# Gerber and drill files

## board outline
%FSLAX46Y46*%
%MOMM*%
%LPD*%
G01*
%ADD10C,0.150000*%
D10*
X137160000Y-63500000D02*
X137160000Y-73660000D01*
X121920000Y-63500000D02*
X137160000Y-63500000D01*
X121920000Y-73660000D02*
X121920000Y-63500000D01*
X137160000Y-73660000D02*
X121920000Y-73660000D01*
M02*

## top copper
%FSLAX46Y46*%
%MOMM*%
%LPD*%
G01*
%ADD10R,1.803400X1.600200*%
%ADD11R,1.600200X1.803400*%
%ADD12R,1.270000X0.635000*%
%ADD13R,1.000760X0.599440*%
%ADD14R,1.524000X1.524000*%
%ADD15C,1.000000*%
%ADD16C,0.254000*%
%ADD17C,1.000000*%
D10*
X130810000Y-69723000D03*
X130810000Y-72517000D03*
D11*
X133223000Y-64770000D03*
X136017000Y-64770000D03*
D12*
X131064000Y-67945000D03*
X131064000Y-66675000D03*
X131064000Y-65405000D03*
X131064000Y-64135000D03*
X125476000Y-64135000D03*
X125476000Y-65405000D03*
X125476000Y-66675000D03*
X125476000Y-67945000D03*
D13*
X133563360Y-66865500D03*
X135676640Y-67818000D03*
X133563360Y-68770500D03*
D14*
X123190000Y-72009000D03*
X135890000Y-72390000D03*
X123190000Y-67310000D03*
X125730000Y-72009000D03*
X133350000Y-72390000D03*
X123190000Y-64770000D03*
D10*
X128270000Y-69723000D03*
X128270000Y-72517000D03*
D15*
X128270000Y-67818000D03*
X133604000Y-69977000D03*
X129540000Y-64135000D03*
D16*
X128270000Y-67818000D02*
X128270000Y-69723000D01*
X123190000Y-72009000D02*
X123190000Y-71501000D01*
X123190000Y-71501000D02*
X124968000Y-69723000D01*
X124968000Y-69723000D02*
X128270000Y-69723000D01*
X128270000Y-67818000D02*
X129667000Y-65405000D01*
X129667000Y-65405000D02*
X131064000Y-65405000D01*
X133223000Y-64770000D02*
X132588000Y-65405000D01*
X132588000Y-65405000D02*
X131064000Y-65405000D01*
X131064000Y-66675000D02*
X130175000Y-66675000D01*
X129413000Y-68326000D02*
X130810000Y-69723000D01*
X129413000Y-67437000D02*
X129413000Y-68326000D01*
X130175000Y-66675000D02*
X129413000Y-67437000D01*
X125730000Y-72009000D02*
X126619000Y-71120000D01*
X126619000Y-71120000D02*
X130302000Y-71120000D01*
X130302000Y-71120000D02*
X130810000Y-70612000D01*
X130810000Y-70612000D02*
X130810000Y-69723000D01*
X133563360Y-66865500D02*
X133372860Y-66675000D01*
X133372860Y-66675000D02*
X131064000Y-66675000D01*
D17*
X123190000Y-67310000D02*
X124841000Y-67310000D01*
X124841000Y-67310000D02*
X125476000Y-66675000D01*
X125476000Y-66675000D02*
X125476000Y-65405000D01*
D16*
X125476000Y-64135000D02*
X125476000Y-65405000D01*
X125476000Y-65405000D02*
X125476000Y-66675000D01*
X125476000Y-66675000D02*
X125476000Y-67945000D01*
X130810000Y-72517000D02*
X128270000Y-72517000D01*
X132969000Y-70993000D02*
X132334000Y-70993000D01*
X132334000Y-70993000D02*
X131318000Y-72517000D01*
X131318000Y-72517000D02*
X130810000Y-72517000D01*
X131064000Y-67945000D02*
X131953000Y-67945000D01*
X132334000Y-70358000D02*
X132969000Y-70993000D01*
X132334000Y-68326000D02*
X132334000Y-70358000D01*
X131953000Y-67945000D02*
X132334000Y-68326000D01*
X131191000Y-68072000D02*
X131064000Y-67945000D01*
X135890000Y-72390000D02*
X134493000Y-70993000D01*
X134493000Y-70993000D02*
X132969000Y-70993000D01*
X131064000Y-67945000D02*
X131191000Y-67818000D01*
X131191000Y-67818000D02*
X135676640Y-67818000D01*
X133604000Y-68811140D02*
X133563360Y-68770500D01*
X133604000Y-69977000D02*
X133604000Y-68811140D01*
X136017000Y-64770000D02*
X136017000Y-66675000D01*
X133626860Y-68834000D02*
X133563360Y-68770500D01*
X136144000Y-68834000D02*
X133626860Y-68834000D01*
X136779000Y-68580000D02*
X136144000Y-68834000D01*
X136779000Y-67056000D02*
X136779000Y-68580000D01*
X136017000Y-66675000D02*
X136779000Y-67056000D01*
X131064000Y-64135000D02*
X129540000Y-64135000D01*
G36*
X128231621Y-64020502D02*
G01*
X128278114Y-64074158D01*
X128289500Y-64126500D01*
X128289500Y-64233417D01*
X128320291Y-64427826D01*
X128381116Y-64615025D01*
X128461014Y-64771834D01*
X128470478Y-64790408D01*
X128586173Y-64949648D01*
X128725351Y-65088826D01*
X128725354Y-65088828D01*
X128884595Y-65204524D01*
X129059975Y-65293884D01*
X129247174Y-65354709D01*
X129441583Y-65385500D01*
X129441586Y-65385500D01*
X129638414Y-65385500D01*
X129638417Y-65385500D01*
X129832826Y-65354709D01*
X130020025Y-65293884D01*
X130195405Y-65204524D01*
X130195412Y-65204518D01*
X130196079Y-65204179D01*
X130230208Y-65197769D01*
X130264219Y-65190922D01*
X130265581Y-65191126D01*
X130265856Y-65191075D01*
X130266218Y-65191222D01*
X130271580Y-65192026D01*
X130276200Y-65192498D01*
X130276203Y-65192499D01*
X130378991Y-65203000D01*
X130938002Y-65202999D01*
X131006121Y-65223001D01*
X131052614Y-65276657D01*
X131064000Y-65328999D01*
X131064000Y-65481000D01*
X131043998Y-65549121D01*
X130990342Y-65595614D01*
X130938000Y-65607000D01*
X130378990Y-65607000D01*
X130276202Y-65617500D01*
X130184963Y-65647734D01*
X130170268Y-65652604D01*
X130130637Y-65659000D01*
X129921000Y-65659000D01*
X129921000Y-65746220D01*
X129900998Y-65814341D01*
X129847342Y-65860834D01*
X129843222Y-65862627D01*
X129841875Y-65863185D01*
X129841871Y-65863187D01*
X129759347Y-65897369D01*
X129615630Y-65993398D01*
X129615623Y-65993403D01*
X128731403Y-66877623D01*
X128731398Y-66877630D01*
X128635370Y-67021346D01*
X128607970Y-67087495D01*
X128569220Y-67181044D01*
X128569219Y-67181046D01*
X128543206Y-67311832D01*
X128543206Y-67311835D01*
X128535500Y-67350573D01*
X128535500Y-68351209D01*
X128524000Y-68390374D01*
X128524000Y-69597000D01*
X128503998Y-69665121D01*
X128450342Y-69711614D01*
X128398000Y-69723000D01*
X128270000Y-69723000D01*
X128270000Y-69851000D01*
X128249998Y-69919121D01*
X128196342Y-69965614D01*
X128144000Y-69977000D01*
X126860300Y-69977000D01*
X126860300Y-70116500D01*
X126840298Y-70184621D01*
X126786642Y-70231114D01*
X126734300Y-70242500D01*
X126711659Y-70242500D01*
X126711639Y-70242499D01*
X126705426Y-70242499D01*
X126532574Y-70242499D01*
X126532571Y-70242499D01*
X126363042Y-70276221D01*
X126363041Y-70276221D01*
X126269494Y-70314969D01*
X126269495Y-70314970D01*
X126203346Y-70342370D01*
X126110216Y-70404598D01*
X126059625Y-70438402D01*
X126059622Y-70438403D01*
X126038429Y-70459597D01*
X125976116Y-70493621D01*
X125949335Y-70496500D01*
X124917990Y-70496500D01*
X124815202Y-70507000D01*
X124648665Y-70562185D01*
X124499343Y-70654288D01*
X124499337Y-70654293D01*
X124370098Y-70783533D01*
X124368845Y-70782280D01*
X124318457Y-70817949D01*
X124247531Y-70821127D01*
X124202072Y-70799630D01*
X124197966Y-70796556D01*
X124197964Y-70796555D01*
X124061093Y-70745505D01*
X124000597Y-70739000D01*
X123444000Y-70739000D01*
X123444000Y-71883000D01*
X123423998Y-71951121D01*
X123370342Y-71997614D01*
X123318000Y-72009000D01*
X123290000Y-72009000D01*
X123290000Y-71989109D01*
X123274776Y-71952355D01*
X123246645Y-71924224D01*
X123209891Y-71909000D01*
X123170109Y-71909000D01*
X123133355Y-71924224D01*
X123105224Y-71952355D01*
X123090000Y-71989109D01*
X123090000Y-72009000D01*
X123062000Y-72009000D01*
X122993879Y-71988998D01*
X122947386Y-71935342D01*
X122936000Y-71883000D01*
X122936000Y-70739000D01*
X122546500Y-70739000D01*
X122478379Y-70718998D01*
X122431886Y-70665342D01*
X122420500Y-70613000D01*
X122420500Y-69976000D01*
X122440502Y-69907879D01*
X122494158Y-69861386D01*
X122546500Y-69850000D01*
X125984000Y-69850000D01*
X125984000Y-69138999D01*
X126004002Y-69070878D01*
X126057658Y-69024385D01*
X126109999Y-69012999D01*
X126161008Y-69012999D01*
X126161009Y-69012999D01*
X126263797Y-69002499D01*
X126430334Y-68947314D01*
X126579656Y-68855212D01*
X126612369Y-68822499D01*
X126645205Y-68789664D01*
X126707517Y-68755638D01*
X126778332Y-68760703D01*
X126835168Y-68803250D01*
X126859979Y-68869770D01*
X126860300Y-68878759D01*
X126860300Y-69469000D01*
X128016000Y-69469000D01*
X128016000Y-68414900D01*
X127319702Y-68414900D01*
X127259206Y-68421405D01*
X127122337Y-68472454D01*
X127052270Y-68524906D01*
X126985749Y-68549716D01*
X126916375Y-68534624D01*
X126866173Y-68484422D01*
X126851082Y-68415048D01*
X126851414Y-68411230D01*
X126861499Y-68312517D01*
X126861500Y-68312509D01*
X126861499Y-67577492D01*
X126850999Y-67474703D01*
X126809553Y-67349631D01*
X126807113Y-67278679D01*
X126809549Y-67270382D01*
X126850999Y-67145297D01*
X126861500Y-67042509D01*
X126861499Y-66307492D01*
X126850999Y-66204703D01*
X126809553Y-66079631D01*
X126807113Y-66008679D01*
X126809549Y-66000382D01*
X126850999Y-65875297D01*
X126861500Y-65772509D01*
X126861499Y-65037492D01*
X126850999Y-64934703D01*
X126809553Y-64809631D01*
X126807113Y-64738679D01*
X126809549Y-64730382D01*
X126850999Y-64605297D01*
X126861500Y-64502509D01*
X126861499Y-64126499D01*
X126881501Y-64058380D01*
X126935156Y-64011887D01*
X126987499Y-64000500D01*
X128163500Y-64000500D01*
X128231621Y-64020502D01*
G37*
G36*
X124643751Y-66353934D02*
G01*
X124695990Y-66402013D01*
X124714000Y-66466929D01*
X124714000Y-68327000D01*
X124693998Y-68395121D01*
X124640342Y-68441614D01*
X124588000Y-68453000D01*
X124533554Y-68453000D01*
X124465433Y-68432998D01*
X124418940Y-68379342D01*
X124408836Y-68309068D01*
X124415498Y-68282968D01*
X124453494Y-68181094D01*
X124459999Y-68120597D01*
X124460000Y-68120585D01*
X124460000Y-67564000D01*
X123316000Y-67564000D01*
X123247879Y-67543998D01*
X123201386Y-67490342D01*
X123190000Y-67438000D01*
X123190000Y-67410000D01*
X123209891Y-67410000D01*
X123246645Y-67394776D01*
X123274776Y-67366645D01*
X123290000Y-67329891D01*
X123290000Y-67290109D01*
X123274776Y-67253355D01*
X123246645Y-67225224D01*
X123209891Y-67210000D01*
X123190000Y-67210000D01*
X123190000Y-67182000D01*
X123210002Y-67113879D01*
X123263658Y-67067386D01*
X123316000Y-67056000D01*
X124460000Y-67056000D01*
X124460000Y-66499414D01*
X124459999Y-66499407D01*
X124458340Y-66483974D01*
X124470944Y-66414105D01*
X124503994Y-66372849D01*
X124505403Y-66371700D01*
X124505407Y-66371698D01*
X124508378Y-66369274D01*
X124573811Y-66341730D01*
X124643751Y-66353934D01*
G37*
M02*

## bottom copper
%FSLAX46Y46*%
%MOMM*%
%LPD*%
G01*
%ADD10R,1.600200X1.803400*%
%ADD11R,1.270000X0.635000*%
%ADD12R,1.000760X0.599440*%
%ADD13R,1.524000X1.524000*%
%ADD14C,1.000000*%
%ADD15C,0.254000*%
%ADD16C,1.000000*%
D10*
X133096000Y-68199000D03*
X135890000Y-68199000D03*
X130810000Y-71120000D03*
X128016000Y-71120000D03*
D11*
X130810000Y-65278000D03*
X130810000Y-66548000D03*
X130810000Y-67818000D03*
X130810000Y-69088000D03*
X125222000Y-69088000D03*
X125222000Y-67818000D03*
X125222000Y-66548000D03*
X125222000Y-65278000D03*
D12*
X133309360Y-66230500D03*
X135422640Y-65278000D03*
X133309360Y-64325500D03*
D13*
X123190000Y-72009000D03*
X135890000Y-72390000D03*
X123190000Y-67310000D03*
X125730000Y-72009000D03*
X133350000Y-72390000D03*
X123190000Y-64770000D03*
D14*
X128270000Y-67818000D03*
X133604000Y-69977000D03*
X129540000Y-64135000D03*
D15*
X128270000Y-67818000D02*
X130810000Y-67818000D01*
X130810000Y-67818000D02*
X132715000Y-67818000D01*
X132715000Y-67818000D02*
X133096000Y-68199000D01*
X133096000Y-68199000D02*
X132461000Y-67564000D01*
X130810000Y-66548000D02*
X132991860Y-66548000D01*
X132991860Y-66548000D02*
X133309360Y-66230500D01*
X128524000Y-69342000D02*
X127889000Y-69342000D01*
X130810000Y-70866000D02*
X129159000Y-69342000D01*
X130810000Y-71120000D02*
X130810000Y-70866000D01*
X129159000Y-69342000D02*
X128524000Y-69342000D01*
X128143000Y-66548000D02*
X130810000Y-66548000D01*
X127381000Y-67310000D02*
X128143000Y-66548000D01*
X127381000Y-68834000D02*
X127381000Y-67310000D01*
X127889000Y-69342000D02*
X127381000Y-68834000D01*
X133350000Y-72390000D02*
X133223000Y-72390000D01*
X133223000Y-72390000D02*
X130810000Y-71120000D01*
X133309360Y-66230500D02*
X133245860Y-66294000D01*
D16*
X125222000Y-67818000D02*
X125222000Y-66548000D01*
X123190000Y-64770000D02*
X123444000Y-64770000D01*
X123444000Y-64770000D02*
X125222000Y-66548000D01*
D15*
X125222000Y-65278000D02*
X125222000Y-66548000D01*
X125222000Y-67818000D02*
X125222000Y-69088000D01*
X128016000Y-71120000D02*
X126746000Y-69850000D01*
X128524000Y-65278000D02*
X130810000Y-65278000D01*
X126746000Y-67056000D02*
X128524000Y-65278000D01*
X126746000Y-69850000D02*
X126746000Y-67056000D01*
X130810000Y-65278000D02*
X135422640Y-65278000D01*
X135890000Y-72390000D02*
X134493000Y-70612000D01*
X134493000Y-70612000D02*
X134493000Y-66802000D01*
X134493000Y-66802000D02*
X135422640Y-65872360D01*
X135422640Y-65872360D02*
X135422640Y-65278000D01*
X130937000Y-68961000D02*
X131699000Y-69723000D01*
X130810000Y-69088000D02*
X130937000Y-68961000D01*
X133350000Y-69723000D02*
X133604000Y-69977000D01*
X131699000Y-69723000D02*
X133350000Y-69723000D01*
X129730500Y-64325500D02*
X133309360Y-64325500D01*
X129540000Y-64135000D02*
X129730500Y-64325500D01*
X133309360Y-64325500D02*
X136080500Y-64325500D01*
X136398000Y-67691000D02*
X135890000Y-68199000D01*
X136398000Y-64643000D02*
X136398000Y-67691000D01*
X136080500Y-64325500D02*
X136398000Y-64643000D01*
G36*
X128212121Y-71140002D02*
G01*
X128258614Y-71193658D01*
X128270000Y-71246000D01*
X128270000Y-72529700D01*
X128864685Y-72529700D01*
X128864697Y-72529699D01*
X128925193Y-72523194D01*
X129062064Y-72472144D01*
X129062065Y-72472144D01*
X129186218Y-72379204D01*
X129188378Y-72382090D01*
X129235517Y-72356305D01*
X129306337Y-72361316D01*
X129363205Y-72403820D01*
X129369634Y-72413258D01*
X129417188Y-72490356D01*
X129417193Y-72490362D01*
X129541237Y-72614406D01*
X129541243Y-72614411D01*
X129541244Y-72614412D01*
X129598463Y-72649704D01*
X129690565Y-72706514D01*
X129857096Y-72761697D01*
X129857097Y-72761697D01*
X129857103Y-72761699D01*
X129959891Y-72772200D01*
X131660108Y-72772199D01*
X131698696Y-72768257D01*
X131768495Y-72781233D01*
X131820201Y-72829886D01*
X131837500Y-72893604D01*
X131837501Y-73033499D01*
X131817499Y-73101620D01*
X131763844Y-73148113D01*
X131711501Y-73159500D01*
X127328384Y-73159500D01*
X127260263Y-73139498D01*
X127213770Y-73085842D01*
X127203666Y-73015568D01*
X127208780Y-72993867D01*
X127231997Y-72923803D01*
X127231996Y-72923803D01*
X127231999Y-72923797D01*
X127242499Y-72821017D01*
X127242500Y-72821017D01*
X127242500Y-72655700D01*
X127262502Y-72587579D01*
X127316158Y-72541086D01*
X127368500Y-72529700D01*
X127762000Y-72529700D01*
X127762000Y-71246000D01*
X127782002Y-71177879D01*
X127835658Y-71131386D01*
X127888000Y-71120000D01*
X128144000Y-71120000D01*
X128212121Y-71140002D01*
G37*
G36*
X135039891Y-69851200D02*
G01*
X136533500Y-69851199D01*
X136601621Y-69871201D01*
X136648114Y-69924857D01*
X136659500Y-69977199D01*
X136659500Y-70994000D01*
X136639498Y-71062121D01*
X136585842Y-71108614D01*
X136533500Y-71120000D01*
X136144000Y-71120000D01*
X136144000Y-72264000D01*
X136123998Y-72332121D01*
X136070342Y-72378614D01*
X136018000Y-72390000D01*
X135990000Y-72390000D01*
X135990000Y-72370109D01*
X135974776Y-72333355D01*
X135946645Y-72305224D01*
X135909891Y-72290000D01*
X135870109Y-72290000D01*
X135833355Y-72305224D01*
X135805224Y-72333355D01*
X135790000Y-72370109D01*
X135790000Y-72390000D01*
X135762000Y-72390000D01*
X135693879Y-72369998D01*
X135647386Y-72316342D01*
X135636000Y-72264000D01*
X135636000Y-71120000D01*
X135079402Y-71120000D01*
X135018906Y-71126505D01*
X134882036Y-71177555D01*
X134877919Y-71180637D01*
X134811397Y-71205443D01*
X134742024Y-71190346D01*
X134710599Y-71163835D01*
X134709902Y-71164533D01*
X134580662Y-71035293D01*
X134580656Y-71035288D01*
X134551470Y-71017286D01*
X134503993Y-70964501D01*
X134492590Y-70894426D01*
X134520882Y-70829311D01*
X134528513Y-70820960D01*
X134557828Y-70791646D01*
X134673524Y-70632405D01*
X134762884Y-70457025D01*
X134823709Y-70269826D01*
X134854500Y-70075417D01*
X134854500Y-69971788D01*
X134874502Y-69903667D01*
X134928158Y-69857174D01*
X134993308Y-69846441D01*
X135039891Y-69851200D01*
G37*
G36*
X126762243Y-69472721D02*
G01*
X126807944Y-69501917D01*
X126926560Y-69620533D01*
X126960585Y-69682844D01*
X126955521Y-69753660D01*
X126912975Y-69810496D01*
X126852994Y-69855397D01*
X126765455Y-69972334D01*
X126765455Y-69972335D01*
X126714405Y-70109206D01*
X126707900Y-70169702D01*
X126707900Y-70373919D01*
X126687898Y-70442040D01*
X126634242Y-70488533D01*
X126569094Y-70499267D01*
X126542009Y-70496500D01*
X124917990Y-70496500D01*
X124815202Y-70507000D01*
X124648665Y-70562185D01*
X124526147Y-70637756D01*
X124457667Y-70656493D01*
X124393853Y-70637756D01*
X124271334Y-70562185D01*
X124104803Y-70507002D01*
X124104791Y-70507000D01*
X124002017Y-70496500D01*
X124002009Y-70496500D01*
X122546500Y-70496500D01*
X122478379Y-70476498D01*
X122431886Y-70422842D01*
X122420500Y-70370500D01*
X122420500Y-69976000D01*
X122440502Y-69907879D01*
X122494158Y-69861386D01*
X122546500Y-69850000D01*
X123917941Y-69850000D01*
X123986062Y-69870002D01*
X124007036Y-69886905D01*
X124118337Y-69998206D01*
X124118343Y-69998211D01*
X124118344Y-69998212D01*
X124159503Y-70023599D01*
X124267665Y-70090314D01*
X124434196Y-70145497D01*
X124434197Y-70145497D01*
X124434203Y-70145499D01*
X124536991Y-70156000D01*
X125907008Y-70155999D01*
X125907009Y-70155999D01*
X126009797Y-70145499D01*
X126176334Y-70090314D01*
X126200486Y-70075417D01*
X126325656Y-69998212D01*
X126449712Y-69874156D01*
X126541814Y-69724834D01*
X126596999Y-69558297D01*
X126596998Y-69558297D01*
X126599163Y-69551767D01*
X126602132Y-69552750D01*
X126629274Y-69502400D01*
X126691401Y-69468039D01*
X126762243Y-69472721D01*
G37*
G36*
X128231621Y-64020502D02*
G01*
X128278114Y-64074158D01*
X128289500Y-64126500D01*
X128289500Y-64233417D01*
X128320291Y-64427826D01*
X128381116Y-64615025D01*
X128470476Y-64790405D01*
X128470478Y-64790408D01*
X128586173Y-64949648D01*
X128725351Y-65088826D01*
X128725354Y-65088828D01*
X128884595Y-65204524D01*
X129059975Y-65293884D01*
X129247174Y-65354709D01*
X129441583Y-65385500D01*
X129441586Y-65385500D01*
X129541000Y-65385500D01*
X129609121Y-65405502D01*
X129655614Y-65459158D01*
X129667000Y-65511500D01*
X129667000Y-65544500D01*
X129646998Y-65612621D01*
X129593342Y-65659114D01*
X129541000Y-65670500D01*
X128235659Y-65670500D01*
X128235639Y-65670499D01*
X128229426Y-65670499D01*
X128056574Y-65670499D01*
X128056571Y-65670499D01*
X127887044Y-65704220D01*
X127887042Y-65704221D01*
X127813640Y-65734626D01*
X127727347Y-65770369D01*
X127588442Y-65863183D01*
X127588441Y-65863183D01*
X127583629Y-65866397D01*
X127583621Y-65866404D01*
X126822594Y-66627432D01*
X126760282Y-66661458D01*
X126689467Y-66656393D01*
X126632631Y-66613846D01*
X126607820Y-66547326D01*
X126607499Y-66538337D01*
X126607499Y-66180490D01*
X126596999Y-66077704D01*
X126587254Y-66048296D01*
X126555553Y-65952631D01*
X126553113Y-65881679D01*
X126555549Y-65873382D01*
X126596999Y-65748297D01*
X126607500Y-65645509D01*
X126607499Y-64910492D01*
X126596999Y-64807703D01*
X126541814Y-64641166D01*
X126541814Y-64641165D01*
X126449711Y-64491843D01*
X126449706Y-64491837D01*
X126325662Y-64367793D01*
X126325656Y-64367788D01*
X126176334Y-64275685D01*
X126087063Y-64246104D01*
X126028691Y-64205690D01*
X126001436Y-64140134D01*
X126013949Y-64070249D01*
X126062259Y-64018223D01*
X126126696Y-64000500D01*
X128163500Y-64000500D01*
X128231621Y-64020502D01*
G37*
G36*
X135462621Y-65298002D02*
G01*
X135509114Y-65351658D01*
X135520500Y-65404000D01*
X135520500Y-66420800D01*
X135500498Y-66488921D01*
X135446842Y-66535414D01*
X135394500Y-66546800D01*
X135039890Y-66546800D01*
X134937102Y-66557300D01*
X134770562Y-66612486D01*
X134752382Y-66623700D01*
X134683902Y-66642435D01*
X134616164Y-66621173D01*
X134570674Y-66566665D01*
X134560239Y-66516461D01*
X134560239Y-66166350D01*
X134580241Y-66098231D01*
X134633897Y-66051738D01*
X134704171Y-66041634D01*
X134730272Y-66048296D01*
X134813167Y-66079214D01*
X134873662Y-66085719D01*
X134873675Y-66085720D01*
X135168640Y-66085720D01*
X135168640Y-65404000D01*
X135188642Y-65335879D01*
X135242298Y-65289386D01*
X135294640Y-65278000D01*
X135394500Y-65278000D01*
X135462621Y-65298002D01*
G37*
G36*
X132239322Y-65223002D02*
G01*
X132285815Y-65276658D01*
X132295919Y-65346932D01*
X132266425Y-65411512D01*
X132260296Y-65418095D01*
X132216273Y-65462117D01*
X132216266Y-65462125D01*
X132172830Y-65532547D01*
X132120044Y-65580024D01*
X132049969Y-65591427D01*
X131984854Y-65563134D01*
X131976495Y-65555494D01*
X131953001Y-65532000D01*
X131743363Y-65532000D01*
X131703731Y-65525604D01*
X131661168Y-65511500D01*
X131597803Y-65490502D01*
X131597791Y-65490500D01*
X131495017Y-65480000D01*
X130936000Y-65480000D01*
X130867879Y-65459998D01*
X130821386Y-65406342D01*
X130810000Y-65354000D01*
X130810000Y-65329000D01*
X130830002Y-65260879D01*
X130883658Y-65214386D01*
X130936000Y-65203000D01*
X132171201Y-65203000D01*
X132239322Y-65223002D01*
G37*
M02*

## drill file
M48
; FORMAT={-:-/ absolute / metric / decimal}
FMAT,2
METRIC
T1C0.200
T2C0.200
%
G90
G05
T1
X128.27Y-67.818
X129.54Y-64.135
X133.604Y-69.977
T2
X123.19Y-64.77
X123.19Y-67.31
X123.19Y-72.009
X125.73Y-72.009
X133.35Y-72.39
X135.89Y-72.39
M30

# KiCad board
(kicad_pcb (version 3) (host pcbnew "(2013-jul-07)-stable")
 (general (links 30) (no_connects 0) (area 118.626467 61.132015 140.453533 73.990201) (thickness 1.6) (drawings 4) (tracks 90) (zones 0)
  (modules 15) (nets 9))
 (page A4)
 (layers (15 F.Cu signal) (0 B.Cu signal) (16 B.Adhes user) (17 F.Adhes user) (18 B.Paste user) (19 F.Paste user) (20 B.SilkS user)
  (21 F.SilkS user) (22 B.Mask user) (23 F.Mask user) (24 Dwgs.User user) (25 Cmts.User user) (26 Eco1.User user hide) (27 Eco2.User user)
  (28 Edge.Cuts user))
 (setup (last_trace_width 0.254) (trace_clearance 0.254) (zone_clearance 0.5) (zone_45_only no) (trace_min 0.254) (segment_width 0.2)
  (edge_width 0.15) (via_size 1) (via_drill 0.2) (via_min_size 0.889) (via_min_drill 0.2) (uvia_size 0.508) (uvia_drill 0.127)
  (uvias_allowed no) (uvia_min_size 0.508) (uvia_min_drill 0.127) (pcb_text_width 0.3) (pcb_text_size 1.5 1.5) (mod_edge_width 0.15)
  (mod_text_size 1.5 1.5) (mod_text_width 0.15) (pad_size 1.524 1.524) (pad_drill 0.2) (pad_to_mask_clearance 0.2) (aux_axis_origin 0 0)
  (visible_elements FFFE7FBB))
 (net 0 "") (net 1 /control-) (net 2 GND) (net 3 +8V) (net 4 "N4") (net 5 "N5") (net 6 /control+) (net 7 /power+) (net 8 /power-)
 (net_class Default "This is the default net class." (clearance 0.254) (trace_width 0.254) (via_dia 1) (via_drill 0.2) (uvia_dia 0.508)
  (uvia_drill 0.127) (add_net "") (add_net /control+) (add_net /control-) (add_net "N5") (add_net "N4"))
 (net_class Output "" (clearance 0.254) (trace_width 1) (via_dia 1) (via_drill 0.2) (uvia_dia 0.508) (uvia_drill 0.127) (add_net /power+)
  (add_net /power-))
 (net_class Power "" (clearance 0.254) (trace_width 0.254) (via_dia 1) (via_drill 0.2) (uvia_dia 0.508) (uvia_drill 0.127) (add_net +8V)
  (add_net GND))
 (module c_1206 (layer F.Cu) (at 130.81 71.12 90)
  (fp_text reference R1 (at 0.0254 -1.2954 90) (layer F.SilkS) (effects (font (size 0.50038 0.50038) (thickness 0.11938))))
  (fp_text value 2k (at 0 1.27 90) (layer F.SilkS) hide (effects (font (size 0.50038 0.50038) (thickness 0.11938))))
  (pad 1 smd rect (at 1.397 0 90) (size 1.6002 1.8034) (layers F.Cu F.Paste F.Mask) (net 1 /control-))
  (pad 2 smd rect (at -1.397 0 90) (size 1.6002 1.8034) (layers F.Cu F.Paste F.Mask) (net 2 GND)))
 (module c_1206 (layer B.Cu) (at 134.493 68.199 180)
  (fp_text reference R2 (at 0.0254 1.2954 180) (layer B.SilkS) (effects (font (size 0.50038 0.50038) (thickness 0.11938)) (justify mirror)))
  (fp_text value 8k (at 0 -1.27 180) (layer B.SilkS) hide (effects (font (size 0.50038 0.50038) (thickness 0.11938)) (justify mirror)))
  (pad 1 smd rect (at 1.397 0 180) (size 1.6002 1.8034) (layers B.Cu B.Paste B.Mask) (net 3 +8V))
  (pad 2 smd rect (at -1.397 0 180) (size 1.6002 1.8034) (layers B.Cu B.Paste B.Mask) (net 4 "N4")))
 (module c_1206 (layer F.Cu) (at 134.62 64.77 180)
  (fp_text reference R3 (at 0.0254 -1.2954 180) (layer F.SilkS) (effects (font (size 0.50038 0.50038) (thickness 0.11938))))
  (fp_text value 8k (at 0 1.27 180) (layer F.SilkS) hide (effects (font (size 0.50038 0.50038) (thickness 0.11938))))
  (pad 1 smd rect (at 1.397 0 180) (size 1.6002 1.8034) (layers F.Cu F.Paste F.Mask) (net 3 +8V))
  (pad 2 smd rect (at -1.397 0 180) (size 1.6002 1.8034) (layers F.Cu F.Paste F.Mask) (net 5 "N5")))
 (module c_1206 (layer B.Cu) (at 129.413 71.12)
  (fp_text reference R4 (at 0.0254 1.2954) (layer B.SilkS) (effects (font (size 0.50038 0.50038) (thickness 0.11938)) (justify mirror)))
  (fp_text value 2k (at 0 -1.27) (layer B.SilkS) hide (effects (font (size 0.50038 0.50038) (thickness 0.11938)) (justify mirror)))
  (pad 1 smd rect (at 1.397 0) (size 1.6002 1.8034) (layers B.Cu B.Paste B.Mask) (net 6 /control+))
  (pad 2 smd rect (at -1.397 0) (size 1.6002 1.8034) (layers B.Cu B.Paste B.Mask) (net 2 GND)))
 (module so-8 (layer F.Cu) (at 128.27 66.04 90)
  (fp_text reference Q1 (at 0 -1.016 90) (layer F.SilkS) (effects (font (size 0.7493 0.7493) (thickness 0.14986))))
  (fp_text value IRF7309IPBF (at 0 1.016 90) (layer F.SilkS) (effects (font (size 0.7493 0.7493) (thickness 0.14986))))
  (pad 1 smd rect (at -1.905 2.794 90) (size 0.635 1.27) (layers F.Cu F.Paste F.Mask) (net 2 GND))
  (pad 2 smd rect (at -0.635 2.794 90) (size 0.635 1.27) (layers F.Cu F.Paste F.Mask) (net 1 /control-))
  (pad 3 smd rect (at 0.635 2.794 90) (size 0.635 1.27) (layers F.Cu F.Paste F.Mask) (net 3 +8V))
  (pad 4 smd rect (at 1.905 2.794 90) (size 0.635 1.27) (layers F.Cu F.Paste F.Mask) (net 4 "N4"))
  (pad 5 smd rect (at 1.905 -2.794 90) (size 0.635 1.27) (layers F.Cu F.Paste F.Mask) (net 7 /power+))
  (pad 6 smd rect (at 0.635 -2.794 90) (size 0.635 1.27) (layers F.Cu F.Paste F.Mask) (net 7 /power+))
  (pad 7 smd rect (at -0.635 -2.794 90) (size 0.635 1.27) (layers F.Cu F.Paste F.Mask) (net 7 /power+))
  (pad 8 smd rect (at -1.905 -2.794 90) (size 0.635 1.27) (layers F.Cu F.Paste F.Mask) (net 7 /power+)))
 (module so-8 (layer B.Cu) (at 128.016 67.183 270)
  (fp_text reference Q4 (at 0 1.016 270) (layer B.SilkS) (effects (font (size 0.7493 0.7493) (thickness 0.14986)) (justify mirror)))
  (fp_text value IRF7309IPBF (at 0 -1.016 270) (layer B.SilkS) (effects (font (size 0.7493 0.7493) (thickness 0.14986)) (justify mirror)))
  (pad 1 smd rect (at -1.905 -2.794 270) (size 0.635 1.27) (layers B.Cu B.Paste B.Mask) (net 2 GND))
  (pad 2 smd rect (at -0.635 -2.794 270) (size 0.635 1.27) (layers B.Cu B.Paste B.Mask) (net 6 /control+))
  (pad 3 smd rect (at 0.635 -2.794 270) (size 0.635 1.27) (layers B.Cu B.Paste B.Mask) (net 3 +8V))
  (pad 4 smd rect (at 1.905 -2.794 270) (size 0.635 1.27) (layers B.Cu B.Paste B.Mask) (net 5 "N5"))
  (pad 5 smd rect (at 1.905 2.794 270) (size 0.635 1.27) (layers B.Cu B.Paste B.Mask) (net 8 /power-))
  (pad 6 smd rect (at 0.635 2.794 270) (size 0.635 1.27) (layers B.Cu B.Paste B.Mask) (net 8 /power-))
  (pad 7 smd rect (at -0.635 2.794 270) (size 0.635 1.27) (layers B.Cu B.Paste B.Mask) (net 8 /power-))
  (pad 8 smd rect (at -1.905 2.794 270) (size 0.635 1.27) (layers B.Cu B.Paste B.Mask) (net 8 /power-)))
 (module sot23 (layer F.Cu) (at 134.62 67.818 270)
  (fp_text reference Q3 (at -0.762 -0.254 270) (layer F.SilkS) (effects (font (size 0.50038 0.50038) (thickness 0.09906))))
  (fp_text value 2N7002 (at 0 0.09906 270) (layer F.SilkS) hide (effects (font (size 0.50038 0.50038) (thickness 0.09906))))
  (pad 1 smd rect (at -0.9525 1.05664 270) (size 0.59944 1.00076) (layers F.Cu F.Paste F.Mask) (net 1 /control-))
  (pad 2 smd rect (at 0 -1.05664 270) (size 0.59944 1.00076) (layers F.Cu F.Paste F.Mask) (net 2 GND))
  (pad 3 smd rect (at 0.9525 1.05664 270) (size 0.59944 1.00076) (layers F.Cu F.Paste F.Mask) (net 5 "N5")))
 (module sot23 (layer B.Cu) (at 134.366 65.278 90)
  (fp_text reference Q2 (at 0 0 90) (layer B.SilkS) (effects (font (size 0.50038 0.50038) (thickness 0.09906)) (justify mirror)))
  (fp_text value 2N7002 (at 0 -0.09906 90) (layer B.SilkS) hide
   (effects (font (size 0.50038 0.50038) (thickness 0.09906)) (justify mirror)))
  (pad 1 smd rect (at -0.9525 -1.05664 90) (size 0.59944 1.00076) (layers B.Cu B.Paste B.Mask) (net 6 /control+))
  (pad 2 smd rect (at 0 1.05664 90) (size 0.59944 1.00076) (layers B.Cu B.Paste B.Mask) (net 2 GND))
  (pad 3 smd rect (at 0.9525 -1.05664 90) (size 0.59944 1.00076) (layers B.Cu B.Paste B.Mask) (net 4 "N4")))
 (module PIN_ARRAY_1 (layer F.Cu) (at 123.19 72.009)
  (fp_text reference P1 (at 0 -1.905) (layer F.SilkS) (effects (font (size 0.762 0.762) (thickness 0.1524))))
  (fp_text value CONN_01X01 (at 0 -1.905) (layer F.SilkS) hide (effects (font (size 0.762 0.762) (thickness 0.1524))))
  (pad 1 thru_hole rect (at 0 0) (size 1.524 1.524) (drill 0.2) (layers *.Cu *.Mask F.SilkS) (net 3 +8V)))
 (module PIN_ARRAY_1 (layer F.Cu) (at 135.89 72.39)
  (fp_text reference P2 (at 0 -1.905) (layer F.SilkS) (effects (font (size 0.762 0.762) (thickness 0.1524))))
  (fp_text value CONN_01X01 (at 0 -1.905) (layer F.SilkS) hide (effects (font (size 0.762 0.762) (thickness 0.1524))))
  (pad 1 thru_hole rect (at 0 0) (size 1.524 1.524) (drill 0.2) (layers *.Cu *.Mask F.SilkS) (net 2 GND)))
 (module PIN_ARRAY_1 (layer F.Cu) (at 123.19 67.31)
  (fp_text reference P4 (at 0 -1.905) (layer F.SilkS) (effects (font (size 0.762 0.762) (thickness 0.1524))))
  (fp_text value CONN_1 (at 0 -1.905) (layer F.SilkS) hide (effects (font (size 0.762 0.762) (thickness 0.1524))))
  (pad 1 thru_hole rect (at 0 0) (size 1.524 1.524) (drill 0.2) (layers *.Cu *.Mask F.SilkS) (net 7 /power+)))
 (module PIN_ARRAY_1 (layer F.Cu) (at 125.73 72.009)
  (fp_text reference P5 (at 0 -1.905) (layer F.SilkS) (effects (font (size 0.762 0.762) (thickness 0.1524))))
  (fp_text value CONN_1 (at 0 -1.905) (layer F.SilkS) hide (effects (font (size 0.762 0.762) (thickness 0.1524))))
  (pad 1 thru_hole rect (at 0 0) (size 1.524 1.524) (drill 0.2) (layers *.Cu *.Mask F.SilkS) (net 1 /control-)))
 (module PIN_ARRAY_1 (layer F.Cu) (at 133.35 72.39)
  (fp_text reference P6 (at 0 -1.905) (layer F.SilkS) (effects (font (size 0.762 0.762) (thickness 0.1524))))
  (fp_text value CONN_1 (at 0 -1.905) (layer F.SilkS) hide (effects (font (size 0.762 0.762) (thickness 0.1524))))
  (pad 1 thru_hole rect (at 0 0) (size 1.524 1.524) (drill 0.2) (layers *.Cu *.Mask F.SilkS) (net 6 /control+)))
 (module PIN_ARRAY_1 (layer F.Cu) (at 123.19 64.77)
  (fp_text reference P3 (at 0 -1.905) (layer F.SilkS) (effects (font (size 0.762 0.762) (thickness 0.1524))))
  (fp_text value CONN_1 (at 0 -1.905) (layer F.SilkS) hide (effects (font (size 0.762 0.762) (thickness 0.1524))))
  (pad 1 thru_hole rect (at 0 0) (size 1.524 1.524) (drill 0.2) (layers *.Cu *.Mask F.SilkS) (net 8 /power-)))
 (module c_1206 (layer F.Cu) (at 128.27 71.12 90)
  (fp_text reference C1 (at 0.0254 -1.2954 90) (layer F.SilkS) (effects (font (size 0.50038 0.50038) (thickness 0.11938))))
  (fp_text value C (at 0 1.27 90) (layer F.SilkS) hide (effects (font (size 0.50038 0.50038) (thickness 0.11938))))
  (pad 1 smd rect (at 1.397 0 90) (size 1.6002 1.8034) (layers F.Cu F.Paste F.Mask) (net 3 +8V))
  (pad 2 smd rect (at -1.397 0 90) (size 1.6002 1.8034) (layers F.Cu F.Paste F.Mask) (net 2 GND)))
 (gr_line (start 137.16 63.5) (end 137.16 73.66) (angle 90) (layer Edge.Cuts) (width 0.15))
 (gr_line (start 121.92 63.5) (end 137.16 63.5) (angle 90) (layer Edge.Cuts) (width 0.15))
 (gr_line (start 121.92 73.66) (end 121.92 63.5) (angle 90) (layer Edge.Cuts) (width 0.15))
 (gr_line (start 137.16 73.66) (end 121.92 73.66) (angle 90) (layer Edge.Cuts) (width 0.15))
 (segment (start 128.27 67.818) (end 128.27 69.723) (width 0.254) (layer F.Cu) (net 3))
 (segment (start 123.19 72.009) (end 123.19 71.501) (width 0.254) (layer F.Cu) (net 3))
 (segment (start 123.19 71.501) (end 124.968 69.723) (width 0.254) (layer F.Cu) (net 3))
 (segment (start 124.968 69.723) (end 128.27 69.723) (width 0.254) (layer F.Cu) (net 3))
 (segment (start 128.27 67.818) (end 130.81 67.818) (width 0.254) (layer B.Cu) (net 3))
 (via (at 128.27 67.818) (size 1) (layers F.Cu B.Cu) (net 3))
 (segment (start 130.81 67.818) (end 132.715 67.818) (width 0.254) (layer B.Cu) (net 3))
 (segment (start 132.715 67.818) (end 133.096 68.199) (width 0.254) (layer B.Cu) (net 3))
 (segment (start 128.27 67.818) (end 129.667 65.405) (width 0.254) (layer F.Cu) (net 3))
 (segment (start 129.667 65.405) (end 131.064 65.405) (width 0.254) (layer F.Cu) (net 3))
 (segment (start 133.223 64.77) (end 132.588 65.405) (width 0.254) (layer F.Cu) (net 3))
 (segment (start 132.588 65.405) (end 131.064 65.405) (width 0.254) (layer F.Cu) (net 3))
 (segment (start 133.096 68.199) (end 132.461 67.564) (width 0.254) (layer B.Cu) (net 3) (status 30))
 (segment (start 130.81 66.548) (end 132.99186 66.548) (width 0.254) (layer B.Cu) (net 6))
 (segment (start 132.99186 66.548) (end 133.30936 66.2305) (width 0.254) (layer B.Cu) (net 6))
 (segment (start 128.524 69.342) (end 127.889 69.342) (width 0.254) (layer B.Cu) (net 6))
 (segment (start 130.81 70.866) (end 129.159 69.342) (width 0.254) (layer B.Cu) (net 6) (status 10))
 (segment (start 130.81 71.12) (end 130.81 70.866) (width 0.254) (layer B.Cu) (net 6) (status 30))
 (segment (start 129.159 69.342) (end 128.524 69.342) (width 0.254) (layer B.Cu) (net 6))
 (segment (start 128.143 66.548) (end 130.81 66.548) (width 0.254) (layer B.Cu) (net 6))
 (segment (start 127.381 67.31) (end 128.143 66.548) (width 0.254) (layer B.Cu) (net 6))
 (segment (start 127.381 68.834) (end 127.381 67.31) (width 0.254) (layer B.Cu) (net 6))
 (segment (start 127.889 69.342) (end 127.381 68.834) (width 0.254) (layer B.Cu) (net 6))
 (segment (start 133.35 72.39) (end 133.223 72.39) (width 0.254) (layer B.Cu) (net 6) (status 30))
 (segment (start 133.223 72.39) (end 130.81 71.12) (width 0.254) (layer B.Cu) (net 6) (status 10))
 (segment (start 133.30936 66.2305) (end 133.24586 66.294) (width 0.254) (layer B.Cu) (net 6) (status 30))
 (segment (start 131.064 66.675) (end 130.175 66.675) (width 0.254) (layer F.Cu) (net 1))
 (segment (start 129.413 68.326) (end 130.81 69.723) (width 0.254) (layer F.Cu) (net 1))
 (segment (start 129.413 67.437) (end 129.413 68.326) (width 0.254) (layer F.Cu) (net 1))
 (segment (start 130.175 66.675) (end 129.413 67.437) (width 0.254) (layer F.Cu) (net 1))
 (segment (start 125.73 72.009) (end 126.619 71.12) (width 0.254) (layer F.Cu) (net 1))
 (segment (start 126.619 71.12) (end 130.302 71.12) (width 0.254) (layer F.Cu) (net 1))
 (segment (start 130.302 71.12) (end 130.81 70.612) (width 0.254) (layer F.Cu) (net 1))
 (segment (start 130.81 70.612) (end 130.81 69.723) (width 0.254) (layer F.Cu) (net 1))
 (segment (start 133.56336 66.8655) (end 133.37286 66.675) (width 0.254) (layer F.Cu) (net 1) (status 30))
 (segment (start 133.37286 66.675) (end 131.064 66.675) (width 0.254) (layer F.Cu) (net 1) (status 10))
 (segment (start 123.19 67.31) (end 124.841 67.31) (width 1) (layer F.Cu) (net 7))
 (segment (start 124.841 67.31) (end 125.476 66.675) (width 1) (layer F.Cu) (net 7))
 (segment (start 125.476 66.675) (end 125.476 65.405) (width 1) (layer F.Cu) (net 7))
 (segment (start 125.476 64.135) (end 125.476 65.405) (width 0.254) (layer F.Cu) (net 7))
 (segment (start 125.476 65.405) (end 125.476 66.675) (width 0.254) (layer F.Cu) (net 7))
 (segment (start 125.476 66.675) (end 125.476 67.945) (width 0.254) (layer F.Cu) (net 7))
 (segment (start 125.222 67.818) (end 125.222 66.548) (width 1) (layer B.Cu) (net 8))
 (segment (start 123.19 64.77) (end 123.444 64.77) (width 1) (layer B.Cu) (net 8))
 (segment (start 123.444 64.77) (end 125.222 66.548) (width 1) (layer B.Cu) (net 8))
 (segment (start 125.222 65.278) (end 125.222 66.548) (width 0.254) (layer B.Cu) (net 8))
 (segment (start 125.222 67.818) (end 125.222 69.088) (width 0.254) (layer B.Cu) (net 8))
 (segment (start 130.81 72.517) (end 128.27 72.517) (width 0.254) (layer F.Cu) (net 2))
 (segment (start 132.969 70.993) (end 132.334 70.993) (width 0.254) (layer F.Cu) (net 2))
 (segment (start 132.334 70.993) (end 131.318 72.517) (width 0.254) (layer F.Cu) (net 2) (status 20))
 (segment (start 131.318 72.517) (end 130.81 72.517) (width 0.254) (layer F.Cu) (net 2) (status 30))
 (segment (start 131.064 67.945) (end 131.953 67.945) (width 0.254) (layer F.Cu) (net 2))
 (segment (start 132.334 70.358) (end 132.969 70.993) (width 0.254) (layer F.Cu) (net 2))
 (segment (start 132.334 68.326) (end 132.334 70.358) (width 0.254) (layer F.Cu) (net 2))
 (segment (start 131.953 67.945) (end 132.334 68.326) (width 0.254) (layer F.Cu) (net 2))
 (segment (start 131.191 68.072) (end 131.064 67.945) (width 0.254) (layer F.Cu) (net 2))
 (segment (start 135.89 72.39) (end 134.493 70.993) (width 0.254) (layer F.Cu) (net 2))
 (segment (start 134.493 70.993) (end 132.969 70.993) (width 0.254) (layer F.Cu) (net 2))
 (segment (start 128.016 71.12) (end 126.746 69.85) (width 0.254) (layer B.Cu) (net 2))
 (segment (start 128.524 65.278) (end 130.81 65.278) (width 0.254) (layer B.Cu) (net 2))
 (segment (start 126.746 67.056) (end 128.524 65.278) (width 0.254) (layer B.Cu) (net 2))
 (segment (start 126.746 69.85) (end 126.746 67.056) (width 0.254) (layer B.Cu) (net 2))
 (segment (start 130.81 65.278) (end 135.42264 65.278) (width 0.254) (layer B.Cu) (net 2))
 (segment (start 135.89 72.39) (end 134.493 70.612) (width 0.254) (layer B.Cu) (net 2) (status 10))
 (segment (start 134.493 70.612) (end 134.493 66.802) (width 0.254) (layer B.Cu) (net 2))
 (segment (start 134.493 66.802) (end 135.42264 65.87236) (width 0.254) (layer B.Cu) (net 2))
 (segment (start 135.42264 65.87236) (end 135.42264 65.278) (width 0.254) (layer B.Cu) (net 2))
 (segment (start 131.064 67.945) (end 131.191 67.818) (width 0.254) (layer F.Cu) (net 2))
 (segment (start 131.191 67.818) (end 135.67664 67.818) (width 0.254) (layer F.Cu) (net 2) (status 20))
 (segment (start 130.937 68.961) (end 131.699 69.723) (width 0.254) (layer B.Cu) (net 5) (status 10))
 (segment (start 130.81 69.088) (end 130.937 68.961) (width 0.254) (layer B.Cu) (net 5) (status 30))
 (segment (start 133.604 68.81114) (end 133.56336 68.7705) (width 0.254) (layer F.Cu) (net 5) (status 30))
 (segment (start 133.604 69.977) (end 133.604 68.81114) (width 0.254) (layer F.Cu) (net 5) (status 20))
 (via (at 133.604 69.977) (size 1) (layers F.Cu B.Cu) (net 5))
 (segment (start 133.35 69.723) (end 133.604 69.977) (width 0.254) (layer B.Cu) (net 5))
 (segment (start 131.699 69.723) (end 133.35 69.723) (width 0.254) (layer B.Cu) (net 5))
 (segment (start 136.017 64.77) (end 136.017 66.675) (width 0.254) (layer F.Cu) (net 5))
 (segment (start 133.62686 68.834) (end 133.56336 68.7705) (width 0.254) (layer F.Cu) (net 5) (status 30))
 (segment (start 136.144 68.834) (end 133.62686 68.834) (width 0.254) (layer F.Cu) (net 5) (status 20))
 (segment (start 136.779 68.58) (end 136.144 68.834) (width 0.254) (layer F.Cu) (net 5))
 (segment (start 136.779 67.056) (end 136.779 68.58) (width 0.254) (layer F.Cu) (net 5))
 (segment (start 136.017 66.675) (end 136.779 67.056) (width 0.254) (layer F.Cu) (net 5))
 (segment (start 131.064 64.135) (end 129.54 64.135) (width 0.254) (layer F.Cu) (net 4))
 (segment (start 129.7305 64.3255) (end 133.30936 64.3255) (width 0.254) (layer B.Cu) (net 4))
 (segment (start 129.54 64.135) (end 129.7305 64.3255) (width 0.254) (layer B.Cu) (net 4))
 (via (at 129.54 64.135) (size 1) (layers F.Cu B.Cu) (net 4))
 (segment (start 133.30936 64.3255) (end 136.0805 64.3255) (width 0.254) (layer B.Cu) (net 4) (status 10))
 (segment (start 136.398 67.691) (end 135.89 68.199) (width 0.254) (layer B.Cu) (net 4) (status 30))
 (segment (start 136.398 64.643) (end 136.398 67.691) (width 0.254) (layer B.Cu) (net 4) (status 20))
 (segment (start 136.0805 64.3255) (end 136.398 64.643) (width 0.254) (layer B.Cu) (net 4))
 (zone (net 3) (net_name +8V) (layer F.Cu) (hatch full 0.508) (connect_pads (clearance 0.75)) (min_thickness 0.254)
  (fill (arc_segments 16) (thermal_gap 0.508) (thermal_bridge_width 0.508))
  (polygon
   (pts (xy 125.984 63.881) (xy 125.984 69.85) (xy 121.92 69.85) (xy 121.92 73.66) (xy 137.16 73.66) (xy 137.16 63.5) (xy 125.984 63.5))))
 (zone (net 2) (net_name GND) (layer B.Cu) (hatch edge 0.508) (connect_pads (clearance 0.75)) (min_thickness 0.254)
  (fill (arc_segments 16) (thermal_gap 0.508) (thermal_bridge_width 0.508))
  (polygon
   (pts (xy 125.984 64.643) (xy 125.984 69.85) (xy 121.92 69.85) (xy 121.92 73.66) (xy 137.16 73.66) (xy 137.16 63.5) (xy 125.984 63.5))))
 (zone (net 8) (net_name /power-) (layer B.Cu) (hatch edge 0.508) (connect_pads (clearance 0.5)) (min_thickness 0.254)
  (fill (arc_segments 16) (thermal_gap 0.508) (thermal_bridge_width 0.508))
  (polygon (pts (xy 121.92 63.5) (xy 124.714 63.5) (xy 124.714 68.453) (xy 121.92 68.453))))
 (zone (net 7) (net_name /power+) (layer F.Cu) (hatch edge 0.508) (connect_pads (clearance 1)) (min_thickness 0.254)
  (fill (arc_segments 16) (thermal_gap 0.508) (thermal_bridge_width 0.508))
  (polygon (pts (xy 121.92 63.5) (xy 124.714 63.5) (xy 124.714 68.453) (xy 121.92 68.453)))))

